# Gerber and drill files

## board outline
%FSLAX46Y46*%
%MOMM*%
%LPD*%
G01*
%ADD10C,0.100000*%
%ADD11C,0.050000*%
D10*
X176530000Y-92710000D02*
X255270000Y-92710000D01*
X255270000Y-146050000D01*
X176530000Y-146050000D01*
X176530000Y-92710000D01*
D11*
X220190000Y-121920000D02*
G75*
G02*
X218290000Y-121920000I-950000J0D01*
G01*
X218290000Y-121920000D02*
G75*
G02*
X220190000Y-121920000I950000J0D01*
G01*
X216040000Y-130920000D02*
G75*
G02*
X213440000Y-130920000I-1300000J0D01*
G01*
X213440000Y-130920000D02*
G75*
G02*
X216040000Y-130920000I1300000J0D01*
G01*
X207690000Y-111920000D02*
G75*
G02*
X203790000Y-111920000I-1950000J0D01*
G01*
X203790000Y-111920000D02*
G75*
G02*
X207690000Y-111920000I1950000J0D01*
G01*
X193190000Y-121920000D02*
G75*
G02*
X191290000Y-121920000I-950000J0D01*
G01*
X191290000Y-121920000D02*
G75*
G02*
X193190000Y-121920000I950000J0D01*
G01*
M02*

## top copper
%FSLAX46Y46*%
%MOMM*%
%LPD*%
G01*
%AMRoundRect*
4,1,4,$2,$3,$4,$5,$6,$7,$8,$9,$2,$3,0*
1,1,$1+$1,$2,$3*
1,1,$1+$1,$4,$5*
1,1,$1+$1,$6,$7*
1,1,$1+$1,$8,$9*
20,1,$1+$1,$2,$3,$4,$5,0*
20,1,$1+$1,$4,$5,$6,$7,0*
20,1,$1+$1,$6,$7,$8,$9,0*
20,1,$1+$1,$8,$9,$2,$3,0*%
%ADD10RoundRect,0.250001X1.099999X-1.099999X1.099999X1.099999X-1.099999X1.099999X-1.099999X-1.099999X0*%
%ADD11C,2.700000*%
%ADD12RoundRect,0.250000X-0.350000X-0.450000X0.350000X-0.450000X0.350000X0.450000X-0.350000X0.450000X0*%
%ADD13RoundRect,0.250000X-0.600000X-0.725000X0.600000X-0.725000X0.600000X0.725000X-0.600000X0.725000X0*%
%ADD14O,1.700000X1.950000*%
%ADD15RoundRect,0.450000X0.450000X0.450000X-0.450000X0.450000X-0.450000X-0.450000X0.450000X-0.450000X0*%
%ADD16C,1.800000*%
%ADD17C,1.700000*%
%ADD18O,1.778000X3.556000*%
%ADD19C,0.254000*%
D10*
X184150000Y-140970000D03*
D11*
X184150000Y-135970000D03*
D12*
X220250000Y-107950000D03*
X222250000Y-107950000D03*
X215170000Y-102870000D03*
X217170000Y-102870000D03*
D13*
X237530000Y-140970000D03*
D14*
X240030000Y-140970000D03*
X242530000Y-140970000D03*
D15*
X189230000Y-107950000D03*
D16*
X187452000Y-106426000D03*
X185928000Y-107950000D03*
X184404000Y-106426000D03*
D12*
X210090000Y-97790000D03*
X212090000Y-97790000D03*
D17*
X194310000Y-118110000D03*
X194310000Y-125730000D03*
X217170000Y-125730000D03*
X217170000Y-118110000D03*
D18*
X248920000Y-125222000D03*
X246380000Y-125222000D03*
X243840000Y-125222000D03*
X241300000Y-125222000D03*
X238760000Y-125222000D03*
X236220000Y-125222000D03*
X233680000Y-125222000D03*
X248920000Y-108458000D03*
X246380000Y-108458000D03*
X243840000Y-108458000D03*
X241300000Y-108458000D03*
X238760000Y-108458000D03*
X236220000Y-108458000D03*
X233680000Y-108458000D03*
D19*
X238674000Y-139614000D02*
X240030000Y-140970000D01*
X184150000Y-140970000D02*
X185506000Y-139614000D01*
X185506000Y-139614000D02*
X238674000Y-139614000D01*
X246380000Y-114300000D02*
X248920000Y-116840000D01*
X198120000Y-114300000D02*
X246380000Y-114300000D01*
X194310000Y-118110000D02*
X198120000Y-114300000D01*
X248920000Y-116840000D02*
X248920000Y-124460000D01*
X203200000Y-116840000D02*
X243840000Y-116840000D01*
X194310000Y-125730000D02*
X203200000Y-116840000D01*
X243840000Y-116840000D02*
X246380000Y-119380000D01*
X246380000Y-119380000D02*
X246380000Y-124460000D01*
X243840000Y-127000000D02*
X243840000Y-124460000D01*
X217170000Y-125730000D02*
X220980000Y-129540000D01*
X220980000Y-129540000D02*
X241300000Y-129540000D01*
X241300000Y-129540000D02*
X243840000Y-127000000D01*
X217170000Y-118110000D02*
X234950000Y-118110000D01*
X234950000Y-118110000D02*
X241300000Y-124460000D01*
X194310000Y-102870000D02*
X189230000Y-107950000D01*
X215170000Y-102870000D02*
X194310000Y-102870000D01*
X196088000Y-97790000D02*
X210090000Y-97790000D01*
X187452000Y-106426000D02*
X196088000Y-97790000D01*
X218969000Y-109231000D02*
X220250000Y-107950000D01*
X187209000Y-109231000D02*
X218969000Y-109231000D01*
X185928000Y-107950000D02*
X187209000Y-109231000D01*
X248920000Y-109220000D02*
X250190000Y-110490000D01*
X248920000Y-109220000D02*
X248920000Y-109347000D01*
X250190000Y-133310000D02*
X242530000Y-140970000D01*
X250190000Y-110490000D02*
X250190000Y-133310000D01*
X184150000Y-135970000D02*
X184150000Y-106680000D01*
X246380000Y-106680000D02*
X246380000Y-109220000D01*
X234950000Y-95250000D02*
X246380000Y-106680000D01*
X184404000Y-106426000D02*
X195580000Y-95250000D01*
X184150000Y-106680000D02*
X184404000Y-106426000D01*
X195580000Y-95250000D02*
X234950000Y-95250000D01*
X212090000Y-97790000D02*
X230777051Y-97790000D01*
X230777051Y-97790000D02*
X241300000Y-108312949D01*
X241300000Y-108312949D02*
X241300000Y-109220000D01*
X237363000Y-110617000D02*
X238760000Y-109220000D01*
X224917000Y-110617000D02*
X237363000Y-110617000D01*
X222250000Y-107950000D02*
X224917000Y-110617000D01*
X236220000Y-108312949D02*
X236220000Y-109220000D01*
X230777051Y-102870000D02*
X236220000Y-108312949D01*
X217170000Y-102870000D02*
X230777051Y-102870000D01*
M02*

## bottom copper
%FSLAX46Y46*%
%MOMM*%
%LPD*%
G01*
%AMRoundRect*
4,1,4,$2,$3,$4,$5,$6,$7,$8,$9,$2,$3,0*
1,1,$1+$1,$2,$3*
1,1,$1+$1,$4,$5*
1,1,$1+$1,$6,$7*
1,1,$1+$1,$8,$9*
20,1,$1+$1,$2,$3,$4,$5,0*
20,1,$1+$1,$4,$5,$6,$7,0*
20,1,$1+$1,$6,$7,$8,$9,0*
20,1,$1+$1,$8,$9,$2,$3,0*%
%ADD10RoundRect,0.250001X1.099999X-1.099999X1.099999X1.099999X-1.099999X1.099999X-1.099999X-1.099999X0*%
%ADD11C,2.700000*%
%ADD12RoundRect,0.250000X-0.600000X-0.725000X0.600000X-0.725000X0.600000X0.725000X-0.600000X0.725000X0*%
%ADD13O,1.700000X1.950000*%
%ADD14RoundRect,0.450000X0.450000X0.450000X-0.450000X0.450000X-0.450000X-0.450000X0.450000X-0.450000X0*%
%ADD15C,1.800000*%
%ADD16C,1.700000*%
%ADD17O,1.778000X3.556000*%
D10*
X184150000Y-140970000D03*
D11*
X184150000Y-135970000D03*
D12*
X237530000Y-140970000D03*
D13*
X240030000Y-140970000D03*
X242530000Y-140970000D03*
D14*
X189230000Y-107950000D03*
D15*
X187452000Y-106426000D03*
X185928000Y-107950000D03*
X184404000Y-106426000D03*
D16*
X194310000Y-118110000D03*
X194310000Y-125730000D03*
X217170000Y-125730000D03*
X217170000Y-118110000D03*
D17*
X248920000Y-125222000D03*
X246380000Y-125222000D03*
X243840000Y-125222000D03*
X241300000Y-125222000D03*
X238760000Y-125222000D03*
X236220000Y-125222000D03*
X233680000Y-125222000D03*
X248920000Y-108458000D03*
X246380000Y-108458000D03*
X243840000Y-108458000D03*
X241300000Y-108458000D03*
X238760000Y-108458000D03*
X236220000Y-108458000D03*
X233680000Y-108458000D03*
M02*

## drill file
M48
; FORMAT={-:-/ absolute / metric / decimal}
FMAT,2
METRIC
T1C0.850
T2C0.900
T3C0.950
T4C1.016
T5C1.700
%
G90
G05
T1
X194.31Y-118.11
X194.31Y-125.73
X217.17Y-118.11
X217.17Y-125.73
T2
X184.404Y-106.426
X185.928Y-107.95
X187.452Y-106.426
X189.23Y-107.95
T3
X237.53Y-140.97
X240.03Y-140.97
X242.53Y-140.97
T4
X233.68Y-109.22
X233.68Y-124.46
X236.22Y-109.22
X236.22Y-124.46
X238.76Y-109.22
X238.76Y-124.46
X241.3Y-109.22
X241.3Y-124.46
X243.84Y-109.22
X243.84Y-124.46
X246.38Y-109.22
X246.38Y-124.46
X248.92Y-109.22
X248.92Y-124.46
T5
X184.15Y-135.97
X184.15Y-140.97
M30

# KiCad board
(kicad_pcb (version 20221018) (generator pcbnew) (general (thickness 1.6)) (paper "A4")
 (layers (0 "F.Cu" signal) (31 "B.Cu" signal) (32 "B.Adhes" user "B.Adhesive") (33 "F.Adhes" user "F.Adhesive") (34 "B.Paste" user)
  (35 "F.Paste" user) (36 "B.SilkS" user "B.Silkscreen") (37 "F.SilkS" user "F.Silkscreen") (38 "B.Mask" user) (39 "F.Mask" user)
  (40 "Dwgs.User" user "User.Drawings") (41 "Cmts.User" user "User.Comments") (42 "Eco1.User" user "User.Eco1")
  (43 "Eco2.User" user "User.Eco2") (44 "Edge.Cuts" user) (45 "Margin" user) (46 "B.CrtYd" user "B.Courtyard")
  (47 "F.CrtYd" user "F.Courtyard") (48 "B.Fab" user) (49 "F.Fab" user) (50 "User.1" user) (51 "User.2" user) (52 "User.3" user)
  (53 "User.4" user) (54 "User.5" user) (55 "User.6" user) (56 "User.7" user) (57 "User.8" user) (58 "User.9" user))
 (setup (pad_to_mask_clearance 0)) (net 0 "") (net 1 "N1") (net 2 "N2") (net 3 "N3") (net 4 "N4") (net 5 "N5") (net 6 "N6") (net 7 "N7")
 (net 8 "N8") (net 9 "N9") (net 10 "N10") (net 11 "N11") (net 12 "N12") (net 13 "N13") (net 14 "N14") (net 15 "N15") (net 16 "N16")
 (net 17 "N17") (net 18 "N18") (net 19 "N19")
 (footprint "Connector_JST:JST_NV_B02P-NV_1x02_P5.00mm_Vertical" (layer "F.Cu") (at 184.15 140.97 90)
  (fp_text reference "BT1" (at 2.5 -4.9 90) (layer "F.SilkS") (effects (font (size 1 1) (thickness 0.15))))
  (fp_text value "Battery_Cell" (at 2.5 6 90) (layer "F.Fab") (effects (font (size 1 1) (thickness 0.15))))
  (pad "1" thru_hole roundrect (at 0 0 90) (size 2.7 2.7) (drill 1.7) (layers "*.Cu" "*.Mask") (roundrect_rratio 0.09259296296) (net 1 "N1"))
  (pad "2" thru_hole circle (at 5 0 90) (size 2.7 2.7) (drill 1.7) (layers "*.Cu" "*.Mask") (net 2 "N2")))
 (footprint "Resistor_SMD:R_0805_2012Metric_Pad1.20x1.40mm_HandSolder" (layer "F.Cu") (at 221.25 107.95)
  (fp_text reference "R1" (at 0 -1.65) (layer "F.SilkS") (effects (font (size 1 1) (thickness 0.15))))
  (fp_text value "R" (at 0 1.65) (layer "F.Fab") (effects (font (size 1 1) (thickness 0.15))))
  (pad "1" smd roundrect (at -1 0) (size 1.2 1.4) (layers "F.Cu" "F.Paste" "F.Mask") (roundrect_rratio 0.2083333333) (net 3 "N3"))
  (pad "2" smd roundrect (at 1 0) (size 1.2 1.4) (layers "F.Cu" "F.Paste" "F.Mask") (roundrect_rratio 0.2083333333) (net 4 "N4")))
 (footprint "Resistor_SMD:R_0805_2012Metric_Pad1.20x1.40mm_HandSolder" (layer "F.Cu") (at 216.17 102.87)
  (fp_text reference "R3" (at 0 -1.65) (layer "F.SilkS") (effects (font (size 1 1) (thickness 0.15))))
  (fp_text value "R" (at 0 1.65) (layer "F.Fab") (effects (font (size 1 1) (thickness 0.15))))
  (pad "1" smd roundrect (at -1 0) (size 1.2 1.4) (layers "F.Cu" "F.Paste" "F.Mask") (roundrect_rratio 0.2083333333) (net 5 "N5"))
  (pad "2" smd roundrect (at 1 0) (size 1.2 1.4) (layers "F.Cu" "F.Paste" "F.Mask") (roundrect_rratio 0.2083333333) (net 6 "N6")))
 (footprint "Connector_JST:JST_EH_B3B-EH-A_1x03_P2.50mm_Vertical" (layer "F.Cu") (at 237.53 140.97)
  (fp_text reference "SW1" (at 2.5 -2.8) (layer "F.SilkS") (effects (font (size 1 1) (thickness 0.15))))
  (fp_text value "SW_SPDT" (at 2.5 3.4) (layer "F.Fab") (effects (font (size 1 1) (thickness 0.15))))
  (pad "1" thru_hole roundrect (at 0 0) (size 1.7 1.95) (drill 0.95) (layers "*.Cu" "*.Mask") (roundrect_rratio 0.1470588235) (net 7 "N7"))
  (pad "2" thru_hole oval (at 2.5 0) (size 1.7 1.95) (drill 0.95) (layers "*.Cu" "*.Mask") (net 1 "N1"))
  (pad "3" thru_hole oval (at 5 0) (size 1.7 1.95) (drill 0.95) (layers "*.Cu" "*.Mask") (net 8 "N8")))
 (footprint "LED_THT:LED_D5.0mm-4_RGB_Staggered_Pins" (layer "F.Cu") (at 189.23 107.95 180)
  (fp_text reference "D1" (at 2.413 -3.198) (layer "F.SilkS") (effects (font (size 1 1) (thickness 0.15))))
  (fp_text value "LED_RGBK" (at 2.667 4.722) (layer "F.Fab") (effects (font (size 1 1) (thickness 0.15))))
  (pad "1" thru_hole roundrect (at 0 0 180) (size 1.8 1.8) (drill 0.9) (layers "*.Cu" "*.Mask") (roundrect_rratio 0.25) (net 5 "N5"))
  (pad "2" thru_hole circle (at 1.778 1.524 180) (size 1.8 1.8) (drill 0.9) (layers "*.Cu" "*.Mask") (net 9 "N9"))
  (pad "3" thru_hole circle (at 3.302 0 180) (size 1.8 1.8) (drill 0.9) (layers "*.Cu" "*.Mask") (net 3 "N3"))
  (pad "4" thru_hole circle (at 4.826 1.524 180) (size 1.8 1.8) (drill 0.9) (layers "*.Cu" "*.Mask") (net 2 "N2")))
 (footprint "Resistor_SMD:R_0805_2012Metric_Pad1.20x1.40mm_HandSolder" (layer "F.Cu") (at 211.09 97.79)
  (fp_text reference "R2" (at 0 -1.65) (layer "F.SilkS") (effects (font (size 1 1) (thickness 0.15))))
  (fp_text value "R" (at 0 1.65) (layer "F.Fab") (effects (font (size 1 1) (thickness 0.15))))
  (pad "1" smd roundrect (at -1 0) (size 1.2 1.4) (layers "F.Cu" "F.Paste" "F.Mask") (roundrect_rratio 0.2083333333) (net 9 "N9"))
  (pad "2" smd roundrect (at 1 0) (size 1.2 1.4) (layers "F.Cu" "F.Paste" "F.Mask") (roundrect_rratio 0.2083333333) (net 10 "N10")))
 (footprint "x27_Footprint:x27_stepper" (layer "B.Cu") (at 203.2 132.08 180)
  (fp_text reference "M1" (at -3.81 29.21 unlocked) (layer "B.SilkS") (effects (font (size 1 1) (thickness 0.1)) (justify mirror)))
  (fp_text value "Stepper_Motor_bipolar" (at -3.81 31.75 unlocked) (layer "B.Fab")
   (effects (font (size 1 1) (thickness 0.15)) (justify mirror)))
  (fp_circle (center -16.04 10.16) (end -15.09 10.16) (stroke (width 0.05) (type default)) (fill none) (layer "Edge.Cuts"))
  (fp_circle (center -11.54 1.16) (end -10.24 1.16) (stroke (width 0.05) (type default)) (fill none) (layer "Edge.Cuts"))
  (fp_circle (center -2.54 20.16) (end -0.59 20.16) (stroke (width 0.05) (type default)) (fill none) (layer "Edge.Cuts"))
  (fp_circle (center 10.96 10.16) (end 11.91 10.16) (stroke (width 0.05) (type default)) (fill none) (layer "Edge.Cuts"))
  (pad "1" thru_hole circle (at 8.89 13.97 180) (size 1.7 1.7) (drill 0.85) (layers "*.Cu" "*.Mask") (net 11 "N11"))
  (pad "2" thru_hole circle (at 8.89 6.35 180) (size 1.7 1.7) (drill 0.85) (layers "*.Cu" "*.Mask") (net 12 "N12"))
  (pad "3" thru_hole circle (at -13.97 6.35 180) (size 1.7 1.7) (drill 0.85) (layers "*.Cu" "*.Mask") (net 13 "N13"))
  (pad "4" thru_hole circle (at -13.97 13.97 180) (size 1.7 1.7) (drill 0.85) (layers "*.Cu" "*.Mask") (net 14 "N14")))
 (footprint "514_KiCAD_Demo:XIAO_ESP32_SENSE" (layer "B.Cu") (at 241.3 116.84 90)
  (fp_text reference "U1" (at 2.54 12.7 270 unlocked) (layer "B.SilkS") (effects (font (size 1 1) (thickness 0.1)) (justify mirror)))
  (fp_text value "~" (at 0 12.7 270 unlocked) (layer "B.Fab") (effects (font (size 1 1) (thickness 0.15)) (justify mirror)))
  (pad "1" thru_hole oval (at -7.62 7.62 90) (size 3.556 1.778) (drill 1.016 (offset -0.762 0)) (layers "*.Cu" "*.Mask") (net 11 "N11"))
  (pad "2" thru_hole oval (at -7.62 5.08 90) (size 3.556 1.778) (drill 1.016 (offset -0.762 0)) (layers "*.Cu" "*.Mask") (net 12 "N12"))
  (pad "3" thru_hole oval (at -7.62 2.54 90) (size 3.556 1.778) (drill 1.016 (offset -0.762 0)) (layers "*.Cu" "*.Mask") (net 13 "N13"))
  (pad "4" thru_hole oval (at -7.62 0 90) (size 3.556 1.778) (drill 1.016 (offset -0.762 0)) (layers "*.Cu" "*.Mask") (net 14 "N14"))
  (pad "5" thru_hole oval (at -7.62 -2.54 90) (size 3.556 1.778) (drill 1.016 (offset -0.762 0)) (layers "*.Cu" "*.Mask") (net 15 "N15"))
  (pad "6" thru_hole oval (at -7.62 -5.08 90) (size 3.556 1.778) (drill 1.016 (offset -0.762 0)) (layers "*.Cu" "*.Mask") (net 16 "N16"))
  (pad "7" thru_hole oval (at -7.62 -7.62 90) (size 3.556 1.778) (drill 1.016 (offset -0.762 0)) (layers "*.Cu" "*.Mask") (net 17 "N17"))
  (pad "8" thru_hole oval (at 7.62 7.62 90) (size 3.556 1.778) (drill 1.016 (offset 0.762 0)) (layers "*.Cu" "*.Mask") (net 8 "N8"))
  (pad "9" thru_hole oval (at 7.62 5.08 90) (size 3.556 1.778) (drill 1.016 (offset 0.762 0)) (layers "*.Cu" "*.Mask") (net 2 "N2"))
  (pad "10" thru_hole oval (at 7.62 2.54 90) (size 3.556 1.778) (drill 1.016 (offset 0.762 0)) (layers "*.Cu" "*.Mask") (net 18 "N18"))
  (pad "11" thru_hole oval (at 7.62 0 90) (size 3.556 1.778) (drill 1.016 (offset 0.762 0)) (layers "*.Cu" "*.Mask") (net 10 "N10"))
  (pad "12" thru_hole oval (at 7.62 -2.54 90) (size 3.556 1.778) (drill 1.016 (offset 0.762 0)) (layers "*.Cu" "*.Mask") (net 4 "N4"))
  (pad "13" thru_hole oval (at 7.62 -5.08 90) (size 3.556 1.778) (drill 1.016 (offset 0.762 0)) (layers "*.Cu" "*.Mask") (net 6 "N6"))
  (pad "14" thru_hole oval (at 7.62 -7.62 90) (size 3.556 1.778) (drill 1.016 (offset 0.762 0)) (layers "*.Cu" "*.Mask") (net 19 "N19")))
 (gr_rect (start 176.53 92.71) (end 255.27 146.05) (stroke (width 0.1) (type default)) (fill none) (layer "Edge.Cuts"))
 (segment (start 238.674 139.614) (end 240.03 140.97) (width 0.254) (layer "F.Cu") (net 1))
 (segment (start 184.15 140.97) (end 185.506 139.614) (width 0.254) (layer "F.Cu") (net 1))
 (segment (start 185.506 139.614) (end 238.674 139.614) (width 0.254) (layer "F.Cu") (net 1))
 (segment (start 246.38 114.3) (end 248.92 116.84) (width 0.254) (layer "F.Cu") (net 11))
 (segment (start 198.12 114.3) (end 246.38 114.3) (width 0.254) (layer "F.Cu") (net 11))
 (segment (start 194.31 118.11) (end 198.12 114.3) (width 0.254) (layer "F.Cu") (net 11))
 (segment (start 248.92 116.84) (end 248.92 124.46) (width 0.254) (layer "F.Cu") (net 11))
 (segment (start 203.2 116.84) (end 243.84 116.84) (width 0.254) (layer "F.Cu") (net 12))
 (segment (start 194.31 125.73) (end 203.2 116.84) (width 0.254) (layer "F.Cu") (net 12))
 (segment (start 243.84 116.84) (end 246.38 119.38) (width 0.254) (layer "F.Cu") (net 12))
 (segment (start 246.38 119.38) (end 246.38 124.46) (width 0.254) (layer "F.Cu") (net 12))
 (segment (start 243.84 127) (end 243.84 124.46) (width 0.254) (layer "F.Cu") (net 13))
 (segment (start 217.17 125.73) (end 220.98 129.54) (width 0.254) (layer "F.Cu") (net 13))
 (segment (start 220.98 129.54) (end 241.3 129.54) (width 0.254) (layer "F.Cu") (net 13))
 (segment (start 241.3 129.54) (end 243.84 127) (width 0.254) (layer "F.Cu") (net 13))
 (segment (start 217.17 118.11) (end 234.95 118.11) (width 0.254) (layer "F.Cu") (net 14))
 (segment (start 234.95 118.11) (end 241.3 124.46) (width 0.254) (layer "F.Cu") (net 14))
 (segment (start 194.31 102.87) (end 189.23 107.95) (width 0.254) (layer "F.Cu") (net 5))
 (segment (start 215.17 102.87) (end 194.31 102.87) (width 0.254) (layer "F.Cu") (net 5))
 (segment (start 196.088 97.79) (end 210.09 97.79) (width 0.254) (layer "F.Cu") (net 9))
 (segment (start 187.452 106.426) (end 196.088 97.79) (width 0.254) (layer "F.Cu") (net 9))
 (segment (start 218.969 109.231) (end 220.25 107.95) (width 0.254) (layer "F.Cu") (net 3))
 (segment (start 187.209 109.231) (end 218.969 109.231) (width 0.254) (layer "F.Cu") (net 3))
 (segment (start 185.928 107.95) (end 187.209 109.231) (width 0.254) (layer "F.Cu") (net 3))
 (segment (start 248.92 109.22) (end 250.19 110.49) (width 0.254) (layer "F.Cu") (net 8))
 (segment (start 248.92 109.22) (end 248.92 109.347) (width 0.254) (layer "F.Cu") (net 8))
 (segment (start 250.19 133.31) (end 242.53 140.97) (width 0.254) (layer "F.Cu") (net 8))
 (segment (start 250.19 110.49) (end 250.19 133.31) (width 0.254) (layer "F.Cu") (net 8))
 (segment (start 184.15 135.97) (end 184.15 106.68) (width 0.254) (layer "F.Cu") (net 2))
 (segment (start 246.38 106.68) (end 246.38 109.22) (width 0.254) (layer "F.Cu") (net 2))
 (segment (start 234.95 95.25) (end 246.38 106.68) (width 0.254) (layer "F.Cu") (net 2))
 (segment (start 184.404 106.426) (end 195.58 95.25) (width 0.254) (layer "F.Cu") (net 2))
 (segment (start 184.15 106.68) (end 184.404 106.426) (width 0.254) (layer "F.Cu") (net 2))
 (segment (start 195.58 95.25) (end 234.95 95.25) (width 0.254) (layer "F.Cu") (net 2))
 (segment (start 212.09 97.79) (end 230.777051 97.79) (width 0.254) (layer "F.Cu") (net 10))
 (segment (start 230.777051 97.79) (end 241.3 108.312949) (width 0.254) (layer "F.Cu") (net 10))
 (segment (start 241.3 108.312949) (end 241.3 109.22) (width 0.254) (layer "F.Cu") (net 10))
 (segment (start 237.363 110.617) (end 238.76 109.22) (width 0.254) (layer "F.Cu") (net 4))
 (segment (start 224.917 110.617) (end 237.363 110.617) (width 0.254) (layer "F.Cu") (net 4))
 (segment (start 222.25 107.95) (end 224.917 110.617) (width 0.254) (layer "F.Cu") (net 4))
 (segment (start 236.22 108.312949) (end 236.22 109.22) (width 0.254) (layer "F.Cu") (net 6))
 (segment (start 230.777051 102.87) (end 236.22 108.312949) (width 0.254) (layer "F.Cu") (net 6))
 (segment (start 217.17 102.87) (end 230.777051 102.87) (width 0.254) (layer "F.Cu") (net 6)))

